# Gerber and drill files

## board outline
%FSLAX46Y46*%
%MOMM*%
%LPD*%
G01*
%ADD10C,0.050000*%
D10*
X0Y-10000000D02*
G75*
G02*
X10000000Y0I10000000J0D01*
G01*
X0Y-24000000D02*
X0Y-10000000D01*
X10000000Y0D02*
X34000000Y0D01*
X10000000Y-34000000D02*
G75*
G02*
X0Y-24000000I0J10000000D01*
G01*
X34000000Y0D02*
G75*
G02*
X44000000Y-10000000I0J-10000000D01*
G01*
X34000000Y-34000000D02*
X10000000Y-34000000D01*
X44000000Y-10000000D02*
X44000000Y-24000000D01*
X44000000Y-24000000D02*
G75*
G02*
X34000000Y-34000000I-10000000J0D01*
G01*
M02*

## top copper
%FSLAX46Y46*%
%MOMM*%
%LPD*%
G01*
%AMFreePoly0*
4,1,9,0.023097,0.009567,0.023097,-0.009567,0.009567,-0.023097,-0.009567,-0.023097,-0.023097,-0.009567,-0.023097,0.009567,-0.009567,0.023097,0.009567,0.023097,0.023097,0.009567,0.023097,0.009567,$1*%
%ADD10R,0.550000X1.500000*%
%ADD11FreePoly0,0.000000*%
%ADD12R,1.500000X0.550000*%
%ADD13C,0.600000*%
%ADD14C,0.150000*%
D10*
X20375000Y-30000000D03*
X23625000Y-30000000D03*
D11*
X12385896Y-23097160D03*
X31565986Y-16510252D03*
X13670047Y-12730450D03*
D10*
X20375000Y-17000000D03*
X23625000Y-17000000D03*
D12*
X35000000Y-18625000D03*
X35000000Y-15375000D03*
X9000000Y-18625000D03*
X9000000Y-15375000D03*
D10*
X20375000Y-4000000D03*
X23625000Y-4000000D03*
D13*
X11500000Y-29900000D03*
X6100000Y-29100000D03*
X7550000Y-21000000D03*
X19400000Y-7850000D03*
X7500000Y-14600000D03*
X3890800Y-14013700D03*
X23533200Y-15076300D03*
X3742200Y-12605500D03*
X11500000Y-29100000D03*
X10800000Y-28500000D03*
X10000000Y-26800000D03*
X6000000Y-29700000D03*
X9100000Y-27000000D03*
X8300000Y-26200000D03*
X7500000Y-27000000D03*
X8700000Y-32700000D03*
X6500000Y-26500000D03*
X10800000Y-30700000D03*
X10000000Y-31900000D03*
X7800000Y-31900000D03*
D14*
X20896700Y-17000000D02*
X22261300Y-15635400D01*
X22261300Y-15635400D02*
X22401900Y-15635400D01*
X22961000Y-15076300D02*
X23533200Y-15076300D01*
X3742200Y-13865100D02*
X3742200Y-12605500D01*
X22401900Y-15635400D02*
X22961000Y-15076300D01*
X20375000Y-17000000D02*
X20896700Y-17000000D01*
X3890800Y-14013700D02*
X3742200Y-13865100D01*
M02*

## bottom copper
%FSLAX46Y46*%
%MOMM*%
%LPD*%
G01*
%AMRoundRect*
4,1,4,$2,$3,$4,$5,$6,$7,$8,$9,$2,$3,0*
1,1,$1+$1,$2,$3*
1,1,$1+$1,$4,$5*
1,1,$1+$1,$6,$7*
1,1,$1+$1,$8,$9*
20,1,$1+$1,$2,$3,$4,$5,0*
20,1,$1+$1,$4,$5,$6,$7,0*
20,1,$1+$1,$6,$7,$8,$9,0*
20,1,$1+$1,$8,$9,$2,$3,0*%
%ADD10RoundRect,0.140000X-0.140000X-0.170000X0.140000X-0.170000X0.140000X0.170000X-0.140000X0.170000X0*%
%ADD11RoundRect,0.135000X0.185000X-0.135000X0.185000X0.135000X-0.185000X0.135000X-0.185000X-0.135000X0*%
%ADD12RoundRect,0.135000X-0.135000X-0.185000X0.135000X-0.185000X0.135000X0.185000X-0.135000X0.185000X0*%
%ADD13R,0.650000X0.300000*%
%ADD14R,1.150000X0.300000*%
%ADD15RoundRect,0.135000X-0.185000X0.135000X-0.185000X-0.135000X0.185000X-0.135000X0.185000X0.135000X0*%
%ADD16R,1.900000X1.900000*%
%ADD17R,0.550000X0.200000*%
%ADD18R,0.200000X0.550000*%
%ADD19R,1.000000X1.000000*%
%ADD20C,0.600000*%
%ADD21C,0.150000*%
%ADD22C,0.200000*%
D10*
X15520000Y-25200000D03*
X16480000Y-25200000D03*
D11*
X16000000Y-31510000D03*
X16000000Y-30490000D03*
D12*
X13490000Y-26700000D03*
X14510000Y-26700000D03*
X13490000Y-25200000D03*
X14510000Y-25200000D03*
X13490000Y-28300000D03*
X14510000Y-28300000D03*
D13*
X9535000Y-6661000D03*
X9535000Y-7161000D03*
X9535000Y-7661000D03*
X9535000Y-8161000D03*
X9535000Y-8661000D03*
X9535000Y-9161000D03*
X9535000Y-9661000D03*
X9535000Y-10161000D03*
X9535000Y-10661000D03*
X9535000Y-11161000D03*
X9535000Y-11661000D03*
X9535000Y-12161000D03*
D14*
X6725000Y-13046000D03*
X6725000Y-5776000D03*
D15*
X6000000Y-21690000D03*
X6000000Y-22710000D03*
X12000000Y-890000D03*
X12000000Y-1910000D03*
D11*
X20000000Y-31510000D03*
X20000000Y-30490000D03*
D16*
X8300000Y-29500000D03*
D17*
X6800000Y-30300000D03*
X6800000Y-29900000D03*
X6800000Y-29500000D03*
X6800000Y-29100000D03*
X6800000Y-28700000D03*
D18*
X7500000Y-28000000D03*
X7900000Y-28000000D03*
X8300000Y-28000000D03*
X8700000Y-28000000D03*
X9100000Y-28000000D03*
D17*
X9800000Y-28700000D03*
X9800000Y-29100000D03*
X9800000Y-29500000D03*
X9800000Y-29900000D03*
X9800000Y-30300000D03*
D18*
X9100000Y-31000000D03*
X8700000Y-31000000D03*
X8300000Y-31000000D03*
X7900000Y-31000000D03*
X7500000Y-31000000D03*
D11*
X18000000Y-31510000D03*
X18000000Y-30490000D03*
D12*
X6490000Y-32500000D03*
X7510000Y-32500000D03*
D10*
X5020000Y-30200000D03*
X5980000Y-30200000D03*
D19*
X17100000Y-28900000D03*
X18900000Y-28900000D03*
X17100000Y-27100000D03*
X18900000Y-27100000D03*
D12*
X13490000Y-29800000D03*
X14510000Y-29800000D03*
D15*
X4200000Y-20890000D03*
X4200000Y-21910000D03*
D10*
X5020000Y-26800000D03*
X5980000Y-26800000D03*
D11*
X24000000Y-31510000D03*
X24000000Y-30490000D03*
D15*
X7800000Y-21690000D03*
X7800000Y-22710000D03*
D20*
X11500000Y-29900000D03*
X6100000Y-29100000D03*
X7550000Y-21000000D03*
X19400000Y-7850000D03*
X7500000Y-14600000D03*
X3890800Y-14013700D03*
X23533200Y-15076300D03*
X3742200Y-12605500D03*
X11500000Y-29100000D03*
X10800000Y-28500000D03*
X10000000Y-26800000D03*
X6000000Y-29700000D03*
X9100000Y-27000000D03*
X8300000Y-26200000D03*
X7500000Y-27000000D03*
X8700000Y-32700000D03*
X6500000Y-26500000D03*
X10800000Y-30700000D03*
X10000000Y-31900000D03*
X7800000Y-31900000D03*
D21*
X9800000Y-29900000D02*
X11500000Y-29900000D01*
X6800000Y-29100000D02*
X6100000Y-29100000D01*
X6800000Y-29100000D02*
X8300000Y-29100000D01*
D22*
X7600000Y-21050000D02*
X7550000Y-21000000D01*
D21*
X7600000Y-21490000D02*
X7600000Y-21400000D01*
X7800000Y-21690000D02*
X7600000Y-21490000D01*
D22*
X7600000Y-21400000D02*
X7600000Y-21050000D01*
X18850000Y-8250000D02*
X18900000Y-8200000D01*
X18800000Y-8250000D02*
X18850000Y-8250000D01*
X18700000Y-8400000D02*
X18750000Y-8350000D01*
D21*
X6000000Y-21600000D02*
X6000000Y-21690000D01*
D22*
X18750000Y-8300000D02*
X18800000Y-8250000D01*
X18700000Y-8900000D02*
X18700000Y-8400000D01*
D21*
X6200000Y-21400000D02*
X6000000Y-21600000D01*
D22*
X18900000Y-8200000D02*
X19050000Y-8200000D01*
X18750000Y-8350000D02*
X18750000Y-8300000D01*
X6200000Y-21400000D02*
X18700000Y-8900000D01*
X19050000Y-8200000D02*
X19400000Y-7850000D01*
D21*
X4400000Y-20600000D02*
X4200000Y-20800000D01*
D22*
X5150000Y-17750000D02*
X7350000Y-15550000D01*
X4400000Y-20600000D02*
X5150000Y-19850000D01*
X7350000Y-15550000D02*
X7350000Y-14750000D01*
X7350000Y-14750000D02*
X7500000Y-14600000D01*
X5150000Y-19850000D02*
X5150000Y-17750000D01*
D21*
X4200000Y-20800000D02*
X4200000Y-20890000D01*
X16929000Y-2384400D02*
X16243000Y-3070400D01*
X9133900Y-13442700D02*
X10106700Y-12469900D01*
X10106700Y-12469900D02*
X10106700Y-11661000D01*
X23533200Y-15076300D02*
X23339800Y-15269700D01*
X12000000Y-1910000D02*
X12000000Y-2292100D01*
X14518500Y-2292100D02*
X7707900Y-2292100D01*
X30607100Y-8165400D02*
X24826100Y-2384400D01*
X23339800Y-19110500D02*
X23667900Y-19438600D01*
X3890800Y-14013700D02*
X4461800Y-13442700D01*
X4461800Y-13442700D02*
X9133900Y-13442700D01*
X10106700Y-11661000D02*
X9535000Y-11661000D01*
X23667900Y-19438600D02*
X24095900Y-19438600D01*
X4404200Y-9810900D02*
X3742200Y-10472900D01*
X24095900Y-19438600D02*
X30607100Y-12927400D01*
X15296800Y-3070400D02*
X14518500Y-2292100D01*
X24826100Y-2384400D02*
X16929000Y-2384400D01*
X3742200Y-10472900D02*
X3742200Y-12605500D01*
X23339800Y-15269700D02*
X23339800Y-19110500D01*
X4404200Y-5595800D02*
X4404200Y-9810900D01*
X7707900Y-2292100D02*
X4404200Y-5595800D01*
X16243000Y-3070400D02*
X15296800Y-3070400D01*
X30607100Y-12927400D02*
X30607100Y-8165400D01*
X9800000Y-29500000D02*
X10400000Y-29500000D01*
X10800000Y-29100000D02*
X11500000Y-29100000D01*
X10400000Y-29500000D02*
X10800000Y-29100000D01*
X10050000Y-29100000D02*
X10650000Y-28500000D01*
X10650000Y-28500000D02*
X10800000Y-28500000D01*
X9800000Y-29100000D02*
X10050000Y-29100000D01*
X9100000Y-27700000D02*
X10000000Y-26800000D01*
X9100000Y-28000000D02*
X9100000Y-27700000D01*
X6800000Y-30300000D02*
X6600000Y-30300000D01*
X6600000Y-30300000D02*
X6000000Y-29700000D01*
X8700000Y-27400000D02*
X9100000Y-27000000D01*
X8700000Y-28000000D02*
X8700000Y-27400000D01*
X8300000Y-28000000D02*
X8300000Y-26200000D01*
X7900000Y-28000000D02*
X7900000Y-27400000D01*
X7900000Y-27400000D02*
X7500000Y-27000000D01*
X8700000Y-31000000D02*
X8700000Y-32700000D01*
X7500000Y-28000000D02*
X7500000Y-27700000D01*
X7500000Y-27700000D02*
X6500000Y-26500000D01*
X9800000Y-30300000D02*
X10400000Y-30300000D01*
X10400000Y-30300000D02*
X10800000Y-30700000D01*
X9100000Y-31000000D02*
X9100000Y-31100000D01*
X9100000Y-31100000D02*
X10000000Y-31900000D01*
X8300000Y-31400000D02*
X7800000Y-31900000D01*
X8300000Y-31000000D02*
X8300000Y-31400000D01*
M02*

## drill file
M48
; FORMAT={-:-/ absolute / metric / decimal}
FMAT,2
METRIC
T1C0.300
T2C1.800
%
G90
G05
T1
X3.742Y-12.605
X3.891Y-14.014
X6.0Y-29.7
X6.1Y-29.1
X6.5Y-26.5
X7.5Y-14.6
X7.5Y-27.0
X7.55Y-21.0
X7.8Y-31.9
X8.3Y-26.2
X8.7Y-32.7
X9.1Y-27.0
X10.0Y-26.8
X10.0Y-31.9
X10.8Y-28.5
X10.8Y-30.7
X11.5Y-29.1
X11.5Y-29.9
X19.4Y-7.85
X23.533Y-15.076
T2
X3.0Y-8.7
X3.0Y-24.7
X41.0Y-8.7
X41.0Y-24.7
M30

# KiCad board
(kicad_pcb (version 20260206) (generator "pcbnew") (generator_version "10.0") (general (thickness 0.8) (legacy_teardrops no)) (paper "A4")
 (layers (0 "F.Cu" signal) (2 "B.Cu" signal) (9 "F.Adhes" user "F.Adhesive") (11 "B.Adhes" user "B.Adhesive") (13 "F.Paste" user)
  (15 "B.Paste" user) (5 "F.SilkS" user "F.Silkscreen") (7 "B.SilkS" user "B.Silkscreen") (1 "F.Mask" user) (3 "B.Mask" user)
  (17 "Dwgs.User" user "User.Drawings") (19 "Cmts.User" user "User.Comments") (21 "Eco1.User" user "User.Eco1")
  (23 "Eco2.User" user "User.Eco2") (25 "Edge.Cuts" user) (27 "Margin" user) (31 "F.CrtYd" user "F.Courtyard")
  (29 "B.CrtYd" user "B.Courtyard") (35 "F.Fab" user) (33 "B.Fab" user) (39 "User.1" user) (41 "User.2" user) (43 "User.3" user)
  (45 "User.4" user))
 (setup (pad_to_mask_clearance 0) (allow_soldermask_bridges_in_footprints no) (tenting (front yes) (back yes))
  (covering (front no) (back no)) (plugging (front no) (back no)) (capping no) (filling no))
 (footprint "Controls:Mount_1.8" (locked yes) (layer "F.Cu") (at 41 24.7)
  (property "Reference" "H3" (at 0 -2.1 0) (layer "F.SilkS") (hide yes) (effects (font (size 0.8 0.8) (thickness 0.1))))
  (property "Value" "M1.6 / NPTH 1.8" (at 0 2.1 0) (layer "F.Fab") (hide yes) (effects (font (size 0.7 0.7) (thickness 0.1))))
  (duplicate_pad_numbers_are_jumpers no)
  (pad "" np_thru_hole circle (at 0 0) (size 1.8 1.8) (drill 1.8) (layers "*.Cu" "*.Mask")))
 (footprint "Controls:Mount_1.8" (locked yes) (layer "F.Cu") (at 3 8.7)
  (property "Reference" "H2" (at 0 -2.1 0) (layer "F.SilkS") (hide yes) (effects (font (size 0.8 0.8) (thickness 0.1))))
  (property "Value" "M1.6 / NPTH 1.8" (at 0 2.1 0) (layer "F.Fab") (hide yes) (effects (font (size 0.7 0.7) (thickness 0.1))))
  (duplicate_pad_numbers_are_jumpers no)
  (pad "" np_thru_hole circle (at 0 0) (size 1.8 1.8) (drill 1.8) (layers "*.Cu" "*.Mask")))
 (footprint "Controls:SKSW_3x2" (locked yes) (layer "F.Cu") (at 22 30)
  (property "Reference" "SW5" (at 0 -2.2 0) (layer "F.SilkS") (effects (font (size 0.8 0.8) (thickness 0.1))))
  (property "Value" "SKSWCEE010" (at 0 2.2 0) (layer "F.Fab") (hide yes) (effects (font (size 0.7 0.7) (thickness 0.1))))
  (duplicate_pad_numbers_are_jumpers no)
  (pad "1" smd rect (at -1.625 0) (size 0.55 1.5) (layers "F.Cu" "F.Mask" "F.Paste") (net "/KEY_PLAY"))
  (pad "2" smd rect (at 1.625 0) (size 0.55 1.5) (layers "F.Cu" "F.Mask" "F.Paste") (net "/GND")))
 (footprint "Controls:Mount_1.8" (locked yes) (layer "F.Cu") (at 41 8.7)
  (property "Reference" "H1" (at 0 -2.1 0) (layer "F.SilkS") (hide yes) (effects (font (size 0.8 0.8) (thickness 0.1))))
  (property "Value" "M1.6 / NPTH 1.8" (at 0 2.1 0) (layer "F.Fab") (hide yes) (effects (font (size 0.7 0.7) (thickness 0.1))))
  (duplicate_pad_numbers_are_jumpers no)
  (pad "" np_thru_hole circle (at 0 0) (size 1.8 1.8) (drill 1.8) (layers "*.Cu" "*.Mask")))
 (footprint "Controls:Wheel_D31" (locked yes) (layer "F.Cu") (at 22 17)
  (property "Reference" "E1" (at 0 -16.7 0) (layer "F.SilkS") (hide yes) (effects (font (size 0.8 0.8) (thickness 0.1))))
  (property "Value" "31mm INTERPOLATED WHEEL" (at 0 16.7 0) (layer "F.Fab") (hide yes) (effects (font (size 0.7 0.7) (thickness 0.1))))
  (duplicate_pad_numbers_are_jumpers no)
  (pad "1" smd custom (at -9.614104 6.09716) (size 0.05 0.05) (layers "F.Cu") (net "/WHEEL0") (options (clearance outline) (anchor circle))
   (primitives))
  (pad "2" smd custom (at 9.565986 -0.489748) (size 0.05 0.05) (layers "F.Cu") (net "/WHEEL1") (options (clearance outline) (anchor circle))
   (primitives))
  (pad "3" smd custom (at -8.329953 -4.26955) (size 0.05 0.05) (layers "F.Cu") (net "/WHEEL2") (options (clearance outline) (anchor circle))
   (primitives)))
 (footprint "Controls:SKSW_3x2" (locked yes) (layer "F.Cu") (at 22 17)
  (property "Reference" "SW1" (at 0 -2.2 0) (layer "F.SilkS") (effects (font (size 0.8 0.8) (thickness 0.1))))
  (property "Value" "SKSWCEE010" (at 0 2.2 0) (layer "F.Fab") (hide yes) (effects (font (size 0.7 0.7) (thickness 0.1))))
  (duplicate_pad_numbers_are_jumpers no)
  (pad "1" smd rect (at -1.625 0) (size 0.55 1.5) (layers "F.Cu" "F.Mask" "F.Paste") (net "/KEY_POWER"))
  (pad "2" smd rect (at 1.625 0) (size 0.55 1.5) (layers "F.Cu" "F.Mask" "F.Paste") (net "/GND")))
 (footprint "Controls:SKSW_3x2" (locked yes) (layer "F.Cu") (at 35 17 90)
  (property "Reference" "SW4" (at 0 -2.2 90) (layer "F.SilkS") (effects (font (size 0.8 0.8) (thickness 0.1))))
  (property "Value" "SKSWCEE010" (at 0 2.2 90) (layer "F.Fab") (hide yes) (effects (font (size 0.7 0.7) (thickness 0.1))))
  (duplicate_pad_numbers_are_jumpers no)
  (pad "1" smd rect (at -1.625 0 90) (size 0.55 1.5) (layers "F.Cu" "F.Mask" "F.Paste") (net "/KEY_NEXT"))
  (pad "2" smd rect (at 1.625 0 90) (size 0.55 1.5) (layers "F.Cu" "F.Mask" "F.Paste") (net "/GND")))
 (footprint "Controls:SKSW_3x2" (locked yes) (layer "F.Cu") (at 9 17 90)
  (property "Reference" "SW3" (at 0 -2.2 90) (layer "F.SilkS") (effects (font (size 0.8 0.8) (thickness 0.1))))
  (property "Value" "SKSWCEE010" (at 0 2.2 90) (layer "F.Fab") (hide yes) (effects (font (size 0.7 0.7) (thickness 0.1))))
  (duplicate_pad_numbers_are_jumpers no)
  (pad "1" smd rect (at -1.625 0 90) (size 0.55 1.5) (layers "F.Cu" "F.Mask" "F.Paste") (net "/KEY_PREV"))
  (pad "2" smd rect (at 1.625 0 90) (size 0.55 1.5) (layers "F.Cu" "F.Mask" "F.Paste") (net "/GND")))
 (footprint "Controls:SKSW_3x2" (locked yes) (layer "F.Cu") (at 22 4)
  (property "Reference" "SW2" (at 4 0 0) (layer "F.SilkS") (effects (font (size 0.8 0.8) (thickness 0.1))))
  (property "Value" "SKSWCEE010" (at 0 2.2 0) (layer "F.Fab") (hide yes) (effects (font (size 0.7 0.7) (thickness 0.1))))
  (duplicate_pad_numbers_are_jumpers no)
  (pad "1" smd rect (at -1.625 0) (size 0.55 1.5) (layers "F.Cu" "F.Mask" "F.Paste") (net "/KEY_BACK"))
  (pad "2" smd rect (at 1.625 0) (size 0.55 1.5) (layers "F.Cu" "F.Mask" "F.Paste") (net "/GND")))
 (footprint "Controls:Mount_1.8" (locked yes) (layer "F.Cu") (at 3 24.7)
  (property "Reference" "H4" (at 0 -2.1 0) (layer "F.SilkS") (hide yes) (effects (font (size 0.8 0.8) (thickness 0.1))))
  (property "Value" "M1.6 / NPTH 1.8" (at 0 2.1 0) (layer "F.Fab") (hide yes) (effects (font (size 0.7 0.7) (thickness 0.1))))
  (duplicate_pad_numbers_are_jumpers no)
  (pad "" np_thru_hole circle (at 0 0) (size 1.8 1.8) (drill 1.8) (layers "*.Cu" "*.Mask")))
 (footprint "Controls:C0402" (layer "B.Cu") (at 16 25.2)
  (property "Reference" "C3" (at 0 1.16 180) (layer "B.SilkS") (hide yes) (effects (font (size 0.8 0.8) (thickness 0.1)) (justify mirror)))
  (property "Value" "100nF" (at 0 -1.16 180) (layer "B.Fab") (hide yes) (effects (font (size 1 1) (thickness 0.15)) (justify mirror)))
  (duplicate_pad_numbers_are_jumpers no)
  (pad "1" smd roundrect (at -0.48 0) (size 0.56 0.62) (layers "B.Cu" "B.Mask" "B.Paste") (roundrect_rratio 0.25) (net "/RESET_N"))
  (pad "2" smd roundrect (at 0.48 0) (size 0.56 0.62) (layers "B.Cu" "B.Mask" "B.Paste") (roundrect_rratio 0.25) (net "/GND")))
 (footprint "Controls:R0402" (layer "B.Cu") (at 16 31 90)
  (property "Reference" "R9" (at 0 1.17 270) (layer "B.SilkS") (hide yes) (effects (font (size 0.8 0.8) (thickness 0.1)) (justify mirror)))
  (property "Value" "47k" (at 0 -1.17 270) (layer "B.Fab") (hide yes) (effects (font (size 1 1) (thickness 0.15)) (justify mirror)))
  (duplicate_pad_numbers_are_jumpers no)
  (pad "1" smd roundrect (at -0.51 0 90) (size 0.54 0.64) (layers "B.Cu" "B.Mask" "B.Paste") (roundrect_rratio 0.25) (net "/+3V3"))
  (pad "2" smd roundrect (at 0.51 0 90) (size 0.54 0.64) (layers "B.Cu" "B.Mask" "B.Paste") (roundrect_rratio 0.25) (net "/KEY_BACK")))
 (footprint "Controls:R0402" (layer "B.Cu") (at 14 26.7)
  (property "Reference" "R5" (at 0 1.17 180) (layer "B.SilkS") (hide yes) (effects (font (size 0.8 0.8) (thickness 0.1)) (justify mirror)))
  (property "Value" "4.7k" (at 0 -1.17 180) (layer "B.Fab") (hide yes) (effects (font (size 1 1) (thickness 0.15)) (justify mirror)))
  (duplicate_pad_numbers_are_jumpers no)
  (pad "1" smd roundrect (at -0.51 0) (size 0.54 0.64) (layers "B.Cu" "B.Mask" "B.Paste") (roundrect_rratio 0.25) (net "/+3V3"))
  (pad "2" smd roundrect (at 0.51 0) (size 0.54 0.64) (layers "B.Cu" "B.Mask" "B.Paste") (roundrect_rratio 0.25) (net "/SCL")))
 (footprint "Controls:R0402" (layer "B.Cu") (at 14 25.2)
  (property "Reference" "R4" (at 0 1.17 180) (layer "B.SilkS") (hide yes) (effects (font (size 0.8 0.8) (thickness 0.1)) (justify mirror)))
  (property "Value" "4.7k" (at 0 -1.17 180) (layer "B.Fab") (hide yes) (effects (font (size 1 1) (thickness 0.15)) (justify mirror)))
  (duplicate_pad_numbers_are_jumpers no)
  (pad "1" smd roundrect (at -0.51 0) (size 0.54 0.64) (layers "B.Cu" "B.Mask" "B.Paste") (roundrect_rratio 0.25) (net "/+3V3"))
  (pad "2" smd roundrect (at 0.51 0) (size 0.54 0.64) (layers "B.Cu" "B.Mask" "B.Paste") (roundrect_rratio 0.25) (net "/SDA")))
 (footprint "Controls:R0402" (layer "B.Cu") (at 14 28.3)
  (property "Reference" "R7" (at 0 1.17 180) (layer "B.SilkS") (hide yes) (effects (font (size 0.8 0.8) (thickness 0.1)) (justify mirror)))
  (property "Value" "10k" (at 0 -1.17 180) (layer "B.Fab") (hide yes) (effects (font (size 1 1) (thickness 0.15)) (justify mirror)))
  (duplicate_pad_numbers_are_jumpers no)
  (pad "1" smd roundrect (at -0.51 0) (size 0.54 0.64) (layers "B.Cu" "B.Mask" "B.Paste") (roundrect_rratio 0.25) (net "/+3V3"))
  (pad "2" smd roundrect (at 0.51 0) (size 0.54 0.64) (layers "B.Cu" "B.Mask" "B.Paste") (roundrect_rratio 0.25) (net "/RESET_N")))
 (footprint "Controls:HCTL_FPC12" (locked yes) (layer "B.Cu") (at 8.13 9.411 -90)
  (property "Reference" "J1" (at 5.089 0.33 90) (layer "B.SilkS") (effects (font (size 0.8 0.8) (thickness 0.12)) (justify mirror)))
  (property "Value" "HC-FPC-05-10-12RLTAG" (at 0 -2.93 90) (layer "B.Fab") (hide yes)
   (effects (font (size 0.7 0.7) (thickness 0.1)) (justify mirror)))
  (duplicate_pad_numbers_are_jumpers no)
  (pad "1" smd rect (at -2.75 -1.405 270) (size 0.3 0.65) (layers "B.Cu" "B.Mask" "B.Paste") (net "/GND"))
  (pad "2" smd rect (at -2.25 -1.405 270) (size 0.3 0.65) (layers "B.Cu" "B.Mask" "B.Paste") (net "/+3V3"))
  (pad "3" smd rect (at -1.75 -1.405 270) (size 0.3 0.65) (layers "B.Cu" "B.Mask" "B.Paste") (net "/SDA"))
  (pad "4" smd rect (at -1.25 -1.405 270) (size 0.3 0.65) (layers "B.Cu" "B.Mask" "B.Paste") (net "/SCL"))
  (pad "5" smd rect (at -0.75 -1.405 270) (size 0.3 0.65) (layers "B.Cu" "B.Mask" "B.Paste") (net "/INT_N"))
  (pad "6" smd rect (at -0.25 -1.405 270) (size 0.3 0.65) (layers "B.Cu" "B.Mask" "B.Paste") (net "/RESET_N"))
  (pad "7" smd rect (at 0.25 -1.405 270) (size 0.3 0.65) (layers "B.Cu" "B.Mask" "B.Paste") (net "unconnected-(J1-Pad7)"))
  (pad "8" smd rect (at 0.75 -1.405 270) (size 0.3 0.65) (layers "B.Cu" "B.Mask" "B.Paste") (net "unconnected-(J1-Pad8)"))
  (pad "9" smd rect (at 1.25 -1.405 270) (size 0.3 0.65) (layers "B.Cu" "B.Mask" "B.Paste") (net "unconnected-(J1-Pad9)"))
  (pad "10" smd rect (at 1.75 -1.405 270) (size 0.3 0.65) (layers "B.Cu" "B.Mask" "B.Paste") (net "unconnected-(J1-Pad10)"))
  (pad "11" smd rect (at 2.25 -1.405 270) (size 0.3 0.65) (layers "B.Cu" "B.Mask" "B.Paste") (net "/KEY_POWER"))
  (pad "12" smd rect (at 2.75 -1.405 270) (size 0.3 0.65) (layers "B.Cu" "B.Mask" "B.Paste") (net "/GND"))
  (pad "13" smd rect (at 3.635 1.405 270) (size 0.3 1.15) (layers "B.Cu" "B.Mask" "B.Paste") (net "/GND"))
  (pad "14" smd rect (at -3.635 1.405 270) (size 0.3 1.15) (layers "B.Cu" "B.Mask" "B.Paste") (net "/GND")))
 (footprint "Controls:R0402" (layer "B.Cu") (at 6 22.2 -90)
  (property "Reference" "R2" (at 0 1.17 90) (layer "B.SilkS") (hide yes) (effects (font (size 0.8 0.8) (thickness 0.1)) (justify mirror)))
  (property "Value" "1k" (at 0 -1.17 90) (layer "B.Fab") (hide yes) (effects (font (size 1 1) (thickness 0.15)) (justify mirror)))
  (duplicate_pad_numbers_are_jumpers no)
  (pad "1" smd roundrect (at -0.51 0 270) (size 0.54 0.64) (layers "B.Cu" "B.Mask" "B.Paste") (roundrect_rratio 0.25) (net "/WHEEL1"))
  (pad "2" smd roundrect (at 0.51 0 270) (size 0.54 0.64) (layers "B.Cu" "B.Mask" "B.Paste") (roundrect_rratio 0.25) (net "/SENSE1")))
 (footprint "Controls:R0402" (layer "B.Cu") (at 12 1.4 -90)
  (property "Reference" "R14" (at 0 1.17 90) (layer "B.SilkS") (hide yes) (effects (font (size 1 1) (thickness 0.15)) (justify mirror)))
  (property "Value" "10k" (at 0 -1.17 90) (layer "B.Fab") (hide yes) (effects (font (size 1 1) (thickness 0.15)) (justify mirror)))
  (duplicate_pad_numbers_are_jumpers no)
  (pad "1" smd roundrect (at -0.51 0 270) (size 0.54 0.64) (layers "B.Cu" "B.Mask" "B.Paste") (roundrect_rratio 0.25) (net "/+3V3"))
  (pad "2" smd roundrect (at 0.51 0 270) (size 0.54 0.64) (layers "B.Cu" "B.Mask" "B.Paste") (roundrect_rratio 0.25) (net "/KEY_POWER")))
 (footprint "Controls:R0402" (layer "B.Cu") (at 20 31 90)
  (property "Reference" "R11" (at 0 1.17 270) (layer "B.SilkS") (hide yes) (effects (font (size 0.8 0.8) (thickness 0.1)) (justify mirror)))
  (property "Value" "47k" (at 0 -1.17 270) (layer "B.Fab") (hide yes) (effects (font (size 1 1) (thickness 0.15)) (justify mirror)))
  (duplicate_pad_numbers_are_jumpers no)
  (pad "1" smd roundrect (at -0.51 0 90) (size 0.54 0.64) (layers "B.Cu" "B.Mask" "B.Paste") (roundrect_rratio 0.25) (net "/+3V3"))
  (pad "2" smd roundrect (at 0.51 0 90) (size 0.54 0.64) (layers "B.Cu" "B.Mask" "B.Paste") (roundrect_rratio 0.25) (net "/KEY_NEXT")))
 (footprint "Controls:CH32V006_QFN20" (layer "B.Cu") (at 8.3 29.5)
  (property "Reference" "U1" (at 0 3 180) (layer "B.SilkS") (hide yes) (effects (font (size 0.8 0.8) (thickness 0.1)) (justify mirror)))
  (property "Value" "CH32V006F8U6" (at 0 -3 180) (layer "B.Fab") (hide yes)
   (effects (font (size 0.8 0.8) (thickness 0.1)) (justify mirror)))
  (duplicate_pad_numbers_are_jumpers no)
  (pad "" smd rect (at -0.45 -0.45) (size 0.7 0.7) (layers "B.Paste"))
  (pad "" smd rect (at -0.45 0.45) (size 0.7 0.7) (layers "B.Paste"))
  (pad "" smd rect (at 0.45 -0.45) (size 0.7 0.7) (layers "B.Paste"))
  (pad "" smd rect (at 0.45 0.45) (size 0.7 0.7) (layers "B.Paste"))
  (pad "0" smd rect (at 0 0) (size 1.9 1.9) (layers "B.Cu" "B.Mask") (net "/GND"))
  (pad "1" smd rect (at -1.5 0.8) (size 0.55 0.2) (layers "B.Cu" "B.Mask" "B.Paste") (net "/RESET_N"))
  (pad "2" smd rect (at -1.5 0.4) (size 0.55 0.2) (layers "B.Cu" "B.Mask" "B.Paste") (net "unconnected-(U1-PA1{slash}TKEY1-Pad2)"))
  (pad "3" smd rect (at -1.5 0) (size 0.55 0.2) (layers "B.Cu" "B.Mask" "B.Paste") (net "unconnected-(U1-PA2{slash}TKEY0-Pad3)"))
  (pad "4" smd rect (at -1.5 -0.4) (size 0.55 0.2) (layers "B.Cu" "B.Mask" "B.Paste") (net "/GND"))
  (pad "5" smd rect (at -1.5 -0.8) (size 0.55 0.2) (layers "B.Cu" "B.Mask" "B.Paste") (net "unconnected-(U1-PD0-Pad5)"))
  (pad "6" smd rect (at -0.8 -1.5) (size 0.2 0.55) (layers "B.Cu" "B.Mask" "B.Paste") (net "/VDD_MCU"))
  (pad "7" smd rect (at -0.4 -1.5) (size 0.2 0.55) (layers "B.Cu" "B.Mask" "B.Paste") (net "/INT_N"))
  (pad "8" smd rect (at 0 -1.5) (size 0.2 0.55) (layers "B.Cu" "B.Mask" "B.Paste") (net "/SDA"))
  (pad "9" smd rect (at 0.4 -1.5) (size 0.2 0.55) (layers "B.Cu" "B.Mask" "B.Paste") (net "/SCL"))
  (pad "10" smd rect (at 0.8 -1.5) (size 0.2 0.55) (layers "B.Cu" "B.Mask" "B.Paste") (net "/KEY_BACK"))
  (pad "11" smd rect (at 1.5 -0.8) (size 0.55 0.2) (layers "B.Cu" "B.Mask" "B.Paste") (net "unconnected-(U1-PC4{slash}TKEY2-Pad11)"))
  (pad "12" smd rect (at 1.5 -0.4) (size 0.55 0.2) (layers "B.Cu" "B.Mask" "B.Paste") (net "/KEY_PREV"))
  (pad "13" smd rect (at 1.5 0) (size 0.55 0.2) (layers "B.Cu" "B.Mask" "B.Paste") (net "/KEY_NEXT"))
  (pad "14" smd rect (at 1.5 0.4) (size 0.55 0.2) (layers "B.Cu" "B.Mask" "B.Paste") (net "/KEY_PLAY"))
  (pad "15" smd rect (at 1.5 0.8) (size 0.55 0.2) (layers "B.Cu" "B.Mask" "B.Paste") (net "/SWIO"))
  (pad "16" smd rect (at 0.8 1.5) (size 0.2 0.55) (layers "B.Cu" "B.Mask" "B.Paste") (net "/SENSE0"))
  (pad "17" smd rect (at 0.4 1.5) (size 0.2 0.55) (layers "B.Cu" "B.Mask" "B.Paste") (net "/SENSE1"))
  (pad "18" smd rect (at 0 1.5) (size 0.2 0.55) (layers "B.Cu" "B.Mask" "B.Paste") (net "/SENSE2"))
  (pad "19" smd rect (at -0.4 1.5) (size 0.2 0.55) (layers "B.Cu" "B.Mask" "B.Paste") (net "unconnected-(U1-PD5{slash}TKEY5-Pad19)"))
  (pad "20" smd rect (at -0.8 1.5) (size 0.2 0.55) (layers "B.Cu" "B.Mask" "B.Paste") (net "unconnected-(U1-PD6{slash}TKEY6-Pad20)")))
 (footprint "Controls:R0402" (layer "B.Cu") (at 18 31 90)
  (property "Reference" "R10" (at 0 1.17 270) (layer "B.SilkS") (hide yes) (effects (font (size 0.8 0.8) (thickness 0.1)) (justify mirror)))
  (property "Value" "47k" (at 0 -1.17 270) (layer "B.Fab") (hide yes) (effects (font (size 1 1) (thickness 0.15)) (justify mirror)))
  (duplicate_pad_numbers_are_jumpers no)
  (pad "1" smd roundrect (at -0.51 0 90) (size 0.54 0.64) (layers "B.Cu" "B.Mask" "B.Paste") (roundrect_rratio 0.25) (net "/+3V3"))
  (pad "2" smd roundrect (at 0.51 0 90) (size 0.54 0.64) (layers "B.Cu" "B.Mask" "B.Paste") (roundrect_rratio 0.25) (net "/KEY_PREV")))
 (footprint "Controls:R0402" (layer "B.Cu") (at 7 32.5)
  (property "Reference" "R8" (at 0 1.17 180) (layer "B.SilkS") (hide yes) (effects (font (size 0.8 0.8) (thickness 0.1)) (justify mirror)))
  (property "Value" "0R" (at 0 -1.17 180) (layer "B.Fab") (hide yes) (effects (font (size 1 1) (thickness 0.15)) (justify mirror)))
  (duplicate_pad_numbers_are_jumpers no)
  (pad "1" smd roundrect (at -0.51 0) (size 0.54 0.64) (layers "B.Cu" "B.Mask" "B.Paste") (roundrect_rratio 0.25) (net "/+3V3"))
  (pad "2" smd roundrect (at 0.51 0) (size 0.54 0.64) (layers "B.Cu" "B.Mask" "B.Paste") (roundrect_rratio 0.25) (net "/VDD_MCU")))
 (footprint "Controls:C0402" (layer "B.Cu") (at 5.5 30.2)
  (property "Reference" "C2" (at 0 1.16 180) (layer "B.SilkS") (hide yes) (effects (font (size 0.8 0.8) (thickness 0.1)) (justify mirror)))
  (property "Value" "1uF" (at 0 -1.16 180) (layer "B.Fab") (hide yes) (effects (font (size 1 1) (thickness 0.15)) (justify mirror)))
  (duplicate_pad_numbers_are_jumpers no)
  (pad "1" smd roundrect (at -0.48 0) (size 0.56 0.62) (layers "B.Cu" "B.Mask" "B.Paste") (roundrect_rratio 0.25) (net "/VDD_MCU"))
  (pad "2" smd roundrect (at 0.48 0) (size 0.56 0.62) (layers "B.Cu" "B.Mask" "B.Paste") (roundrect_rratio 0.25) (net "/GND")))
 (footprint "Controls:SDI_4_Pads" (layer "B.Cu") (at 18 28)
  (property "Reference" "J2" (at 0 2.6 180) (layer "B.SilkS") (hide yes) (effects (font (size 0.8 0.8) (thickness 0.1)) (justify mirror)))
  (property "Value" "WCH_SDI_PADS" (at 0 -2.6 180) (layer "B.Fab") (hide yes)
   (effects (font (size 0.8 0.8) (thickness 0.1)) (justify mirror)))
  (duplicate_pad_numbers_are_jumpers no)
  (pad "1" smd rect (at -0.9 0.9) (size 1 1) (layers "B.Cu" "B.Mask") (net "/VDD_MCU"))
  (pad "2" smd rect (at 0.9 0.9) (size 1 1) (layers "B.Cu" "B.Mask") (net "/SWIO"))
  (pad "3" smd rect (at -0.9 -0.9) (size 1 1) (layers "B.Cu" "B.Mask") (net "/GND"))
  (pad "4" smd rect (at 0.9 -0.9) (size 1 1) (layers "B.Cu" "B.Mask") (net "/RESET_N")))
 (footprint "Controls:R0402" (layer "B.Cu") (at 14 29.8)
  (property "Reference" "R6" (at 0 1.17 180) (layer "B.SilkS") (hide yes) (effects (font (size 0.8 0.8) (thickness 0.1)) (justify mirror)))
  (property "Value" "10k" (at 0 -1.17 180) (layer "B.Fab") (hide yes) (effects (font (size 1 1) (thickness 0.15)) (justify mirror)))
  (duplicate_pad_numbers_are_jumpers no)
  (pad "1" smd roundrect (at -0.51 0) (size 0.54 0.64) (layers "B.Cu" "B.Mask" "B.Paste") (roundrect_rratio 0.25) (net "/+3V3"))
  (pad "2" smd roundrect (at 0.51 0) (size 0.54 0.64) (layers "B.Cu" "B.Mask" "B.Paste") (roundrect_rratio 0.25) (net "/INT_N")))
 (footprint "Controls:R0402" (layer "B.Cu") (at 4.2 21.4 -90)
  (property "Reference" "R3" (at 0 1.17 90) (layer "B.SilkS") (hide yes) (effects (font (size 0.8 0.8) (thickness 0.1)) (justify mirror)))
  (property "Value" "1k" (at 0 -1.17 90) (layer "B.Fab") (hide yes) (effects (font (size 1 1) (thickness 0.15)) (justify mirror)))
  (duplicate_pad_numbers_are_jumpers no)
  (pad "1" smd roundrect (at -0.51 0 270) (size 0.54 0.64) (layers "B.Cu" "B.Mask" "B.Paste") (roundrect_rratio 0.25) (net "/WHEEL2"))
  (pad "2" smd roundrect (at 0.51 0 270) (size 0.54 0.64) (layers "B.Cu" "B.Mask" "B.Paste") (roundrect_rratio 0.25) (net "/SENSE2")))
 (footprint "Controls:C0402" (layer "B.Cu") (at 5.5 26.8)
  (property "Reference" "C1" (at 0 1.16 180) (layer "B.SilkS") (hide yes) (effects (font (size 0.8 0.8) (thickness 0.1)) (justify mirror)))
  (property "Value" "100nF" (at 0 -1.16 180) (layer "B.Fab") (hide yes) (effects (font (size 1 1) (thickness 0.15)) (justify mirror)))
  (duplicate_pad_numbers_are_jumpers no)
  (pad "1" smd roundrect (at -0.48 0) (size 0.56 0.62) (layers "B.Cu" "B.Mask" "B.Paste") (roundrect_rratio 0.25) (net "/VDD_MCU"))
  (pad "2" smd roundrect (at 0.48 0) (size 0.56 0.62) (layers "B.Cu" "B.Mask" "B.Paste") (roundrect_rratio 0.25) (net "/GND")))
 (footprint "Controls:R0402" (layer "B.Cu") (at 24 31 90)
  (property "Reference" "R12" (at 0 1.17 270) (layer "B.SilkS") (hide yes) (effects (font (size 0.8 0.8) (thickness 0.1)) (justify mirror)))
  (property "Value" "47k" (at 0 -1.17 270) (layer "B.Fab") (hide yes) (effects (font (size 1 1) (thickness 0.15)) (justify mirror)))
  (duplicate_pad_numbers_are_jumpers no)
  (pad "1" smd roundrect (at -0.51 0 90) (size 0.54 0.64) (layers "B.Cu" "B.Mask" "B.Paste") (roundrect_rratio 0.25) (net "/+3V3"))
  (pad "2" smd roundrect (at 0.51 0 90) (size 0.54 0.64) (layers "B.Cu" "B.Mask" "B.Paste") (roundrect_rratio 0.25) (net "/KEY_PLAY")))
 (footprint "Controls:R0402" (layer "B.Cu") (at 7.8 22.2 -90)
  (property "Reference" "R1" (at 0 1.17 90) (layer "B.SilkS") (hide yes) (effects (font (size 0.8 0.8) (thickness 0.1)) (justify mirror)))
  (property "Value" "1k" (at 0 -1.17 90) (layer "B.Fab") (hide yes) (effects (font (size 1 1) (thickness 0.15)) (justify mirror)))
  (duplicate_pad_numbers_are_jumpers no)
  (pad "1" smd roundrect (at -0.51 0 270) (size 0.54 0.64) (layers "B.Cu" "B.Mask" "B.Paste") (roundrect_rratio 0.25) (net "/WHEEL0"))
  (pad "2" smd roundrect (at 0.51 0 270) (size 0.54 0.64) (layers "B.Cu" "B.Mask" "B.Paste") (roundrect_rratio 0.25) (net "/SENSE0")))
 (gr_arc (start 0 10) (mid 2.928932 2.928932) (end 10 0) (stroke (width 0.05) (type default)) (layer "Edge.Cuts"))
 (gr_line (start 0 24) (end 0 10) (stroke (width 0.05) (type default)) (layer "Edge.Cuts"))
 (gr_line (start 10 0) (end 34 0) (stroke (width 0.05) (type default)) (layer "Edge.Cuts"))
 (gr_arc (start 10 34) (mid 2.928932 31.071068) (end 0 24) (stroke (width 0.05) (type default)) (layer "Edge.Cuts"))
 (gr_arc (start 34 0) (mid 41.071068 2.928932) (end 44 10) (stroke (width 0.05) (type default)) (layer "Edge.Cuts"))
 (gr_line (start 34 34) (end 10 34) (stroke (width 0.05) (type default)) (layer "Edge.Cuts"))
 (gr_line (start 44 10) (end 44 24) (stroke (width 0.05) (type default)) (layer "Edge.Cuts"))
 (gr_arc (start 44 24) (mid 41.071068 31.071068) (end 34 34) (stroke (width 0.05) (type default)) (layer "Edge.Cuts"))
 (via (at 11.5 29.9) (size 0.6) (drill 0.3) (layers "F.Cu" "B.Cu") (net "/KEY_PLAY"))
 (segment (start 9.8 29.9) (end 11.5 29.9) (width 0.15) (layer "B.Cu") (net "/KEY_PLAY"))
 (via (at 6.1 29.1) (size 0.6) (drill 0.3) (layers "F.Cu" "B.Cu") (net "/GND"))
 (segment (start 6.8 29.1) (end 6.1 29.1) (width 0.15) (layer "B.Cu") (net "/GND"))
 (segment (start 6.8 29.1) (end 8.3 29.1) (width 0.15) (layer "B.Cu") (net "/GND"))
 (via (at 7.55 21) (size 0.6) (drill 0.3) (layers "F.Cu" "B.Cu") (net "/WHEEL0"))
 (segment (start 7.6 21.05) (end 7.55 21) (width 0.2) (layer "B.Cu") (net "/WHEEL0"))
 (segment (start 7.6 21.49) (end 7.6 21.4) (width 0.15) (layer "B.Cu") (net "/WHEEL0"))
 (segment (start 7.8 21.69) (end 7.6 21.49) (width 0.15) (layer "B.Cu") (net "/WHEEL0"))
 (segment (start 7.6 21.4) (end 7.6 21.05) (width 0.2) (layer "B.Cu") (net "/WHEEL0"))
 (via (at 19.4 7.85) (size 0.6) (drill 0.3) (layers "F.Cu" "B.Cu") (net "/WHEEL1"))
 (segment (start 18.85 8.25) (end 18.9 8.2) (width 0.2) (layer "B.Cu") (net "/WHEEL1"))
 (segment (start 18.8 8.25) (end 18.85 8.25) (width 0.2) (layer "B.Cu") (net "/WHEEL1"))
 (segment (start 18.7 8.4) (end 18.75 8.35) (width 0.2) (layer "B.Cu") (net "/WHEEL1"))
 (segment (start 6 21.6) (end 6 21.69) (width 0.15) (layer "B.Cu") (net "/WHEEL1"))
 (segment (start 18.75 8.3) (end 18.8 8.25) (width 0.2) (layer "B.Cu") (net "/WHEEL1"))
 (segment (start 18.7 8.9) (end 18.7 8.4) (width 0.2) (layer "B.Cu") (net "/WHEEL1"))
 (segment (start 6.2 21.4) (end 6 21.6) (width 0.15) (layer "B.Cu") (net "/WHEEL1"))
 (segment (start 18.9 8.2) (end 19.05 8.2) (width 0.2) (layer "B.Cu") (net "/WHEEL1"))
 (segment (start 18.75 8.35) (end 18.75 8.3) (width 0.2) (layer "B.Cu") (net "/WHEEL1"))
 (segment (start 6.2 21.4) (end 18.7 8.9) (width 0.2) (layer "B.Cu") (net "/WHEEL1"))
 (segment (start 19.05 8.2) (end 19.4 7.85) (width 0.2) (layer "B.Cu") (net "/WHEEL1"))
 (via (at 7.5 14.6) (size 0.6) (drill 0.3) (layers "F.Cu" "B.Cu") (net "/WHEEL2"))
 (segment (start 4.4 20.6) (end 4.2 20.8) (width 0.15) (layer "B.Cu") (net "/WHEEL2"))
 (segment (start 5.15 17.75) (end 7.35 15.55) (width 0.2) (layer "B.Cu") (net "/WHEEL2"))
 (segment (start 4.4 20.6) (end 5.15 19.85) (width 0.2) (layer "B.Cu") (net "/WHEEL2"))
 (segment (start 7.35 15.55) (end 7.35 14.75) (width 0.2) (layer "B.Cu") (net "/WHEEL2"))
 (segment (start 7.35 14.75) (end 7.5 14.6) (width 0.2) (layer "B.Cu") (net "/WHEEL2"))
 (segment (start 5.15 19.85) (end 5.15 17.75) (width 0.2) (layer "B.Cu") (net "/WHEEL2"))
 (segment (start 4.2 20.8) (end 4.2 20.89) (width 0.15) (layer "B.Cu") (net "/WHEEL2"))
 (segment (start 20.8967 17) (end 22.2613 15.6354) (width 0.15) (layer "F.Cu") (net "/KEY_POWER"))
 (segment (start 22.2613 15.6354) (end 22.4019 15.6354) (width 0.15) (layer "F.Cu") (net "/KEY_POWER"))
 (segment (start 22.961 15.0763) (end 23.5332 15.0763) (width 0.15) (layer "F.Cu") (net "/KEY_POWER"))
 (segment (start 3.7422 13.8651) (end 3.7422 12.6055) (width 0.15) (layer "F.Cu") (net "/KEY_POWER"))
 (segment (start 22.4019 15.6354) (end 22.961 15.0763) (width 0.15) (layer "F.Cu") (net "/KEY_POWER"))
 (segment (start 20.375 17) (end 20.8967 17) (width 0.15) (layer "F.Cu") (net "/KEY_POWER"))
 (segment (start 3.8908 14.0137) (end 3.7422 13.8651) (width 0.15) (layer "F.Cu") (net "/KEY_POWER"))
 (via (at 3.8908 14.0137) (size 0.6) (drill 0.3) (layers "F.Cu" "B.Cu") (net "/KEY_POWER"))
 (via (at 23.5332 15.0763) (size 0.6) (drill 0.3) (layers "F.Cu" "B.Cu") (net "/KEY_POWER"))
 (via (at 3.7422 12.6055) (size 0.6) (drill 0.3) (layers "F.Cu" "B.Cu") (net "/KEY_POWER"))
 (segment (start 16.929 2.3844) (end 16.243 3.0704) (width 0.15) (layer "B.Cu") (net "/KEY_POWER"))
 (segment (start 9.1339 13.4427) (end 10.1067 12.4699) (width 0.15) (layer "B.Cu") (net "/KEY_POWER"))
 (segment (start 10.1067 12.4699) (end 10.1067 11.661) (width 0.15) (layer "B.Cu") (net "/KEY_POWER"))
 (segment (start 23.5332 15.0763) (end 23.3398 15.2697) (width 0.15) (layer "B.Cu") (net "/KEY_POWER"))
 (segment (start 12 1.91) (end 12 2.2921) (width 0.15) (layer "B.Cu") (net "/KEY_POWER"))
 (segment (start 14.5185 2.2921) (end 7.7079 2.2921) (width 0.15) (layer "B.Cu") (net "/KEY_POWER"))
 (segment (start 30.6071 8.1654) (end 24.8261 2.3844) (width 0.15) (layer "B.Cu") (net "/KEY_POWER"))
 (segment (start 23.3398 19.1105) (end 23.6679 19.4386) (width 0.15) (layer "B.Cu") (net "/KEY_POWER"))
 (segment (start 3.8908 14.0137) (end 4.4618 13.4427) (width 0.15) (layer "B.Cu") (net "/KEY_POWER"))
 (segment (start 4.4618 13.4427) (end 9.1339 13.4427) (width 0.15) (layer "B.Cu") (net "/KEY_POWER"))
 (segment (start 10.1067 11.661) (end 9.535 11.661) (width 0.15) (layer "B.Cu") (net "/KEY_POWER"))
 (segment (start 23.6679 19.4386) (end 24.0959 19.4386) (width 0.15) (layer "B.Cu") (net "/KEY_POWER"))
 (segment (start 4.4042 9.8109) (end 3.7422 10.4729) (width 0.15) (layer "B.Cu") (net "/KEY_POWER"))
 (segment (start 24.0959 19.4386) (end 30.6071 12.9274) (width 0.15) (layer "B.Cu") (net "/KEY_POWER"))
 (segment (start 15.2968 3.0704) (end 14.5185 2.2921) (width 0.15) (layer "B.Cu") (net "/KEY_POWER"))
 (segment (start 24.8261 2.3844) (end 16.929 2.3844) (width 0.15) (layer "B.Cu") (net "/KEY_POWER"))
 (segment (start 3.7422 10.4729) (end 3.7422 12.6055) (width 0.15) (layer "B.Cu") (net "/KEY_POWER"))
 (segment (start 23.3398 15.2697) (end 23.3398 19.1105) (width 0.15) (layer "B.Cu") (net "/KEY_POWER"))
 (segment (start 4.4042 5.5958) (end 4.4042 9.8109) (width 0.15) (layer "B.Cu") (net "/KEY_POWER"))
 (segment (start 7.7079 2.2921) (end 4.4042 5.5958) (width 0.15) (layer "B.Cu") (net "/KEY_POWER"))
 (segment (start 16.243 3.0704) (end 15.2968 3.0704) (width 0.15) (layer "B.Cu") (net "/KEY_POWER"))
 (segment (start 30.6071 12.9274) (end 30.6071 8.1654) (width 0.15) (layer "B.Cu") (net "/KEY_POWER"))
 (via (at 11.5 29.1) (size 0.6) (drill 0.3) (layers "F.Cu" "B.Cu") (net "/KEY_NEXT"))
 (segment (start 9.8 29.5) (end 10.4 29.5) (width 0.15) (layer "B.Cu") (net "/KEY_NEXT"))
 (segment (start 10.8 29.1) (end 11.5 29.1) (width 0.15) (layer "B.Cu") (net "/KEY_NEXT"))
 (segment (start 10.4 29.5) (end 10.8 29.1) (width 0.15) (layer "B.Cu") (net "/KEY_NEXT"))
 (via (at 10.8 28.5) (size 0.6) (drill 0.3) (layers "F.Cu" "B.Cu") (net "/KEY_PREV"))
 (segment (start 10.05 29.1) (end 10.65 28.5) (width 0.15) (layer "B.Cu") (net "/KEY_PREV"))
 (segment (start 10.65 28.5) (end 10.8 28.5) (width 0.15) (layer "B.Cu") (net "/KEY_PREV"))
 (segment (start 9.8 29.1) (end 10.05 29.1) (width 0.15) (layer "B.Cu") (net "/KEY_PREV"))
 (via (at 10 26.8) (size 0.6) (drill 0.3) (layers "F.Cu" "B.Cu") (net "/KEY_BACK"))
 (segment (start 9.1 27.7) (end 10 26.8) (width 0.15) (layer "B.Cu") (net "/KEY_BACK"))
 (segment (start 9.1 28) (end 9.1 27.7) (width 0.15) (layer "B.Cu") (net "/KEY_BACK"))
 (via (at 6 29.7) (size 0.6) (drill 0.3) (layers "F.Cu" "B.Cu") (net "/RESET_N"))
 (segment (start 6.8 30.3) (end 6.6 30.3) (width 0.15) (layer "B.Cu") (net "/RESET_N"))
 (segment (start 6.6 30.3) (end 6 29.7) (width 0.15) (layer "B.Cu") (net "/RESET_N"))
 (via (at 9.1 27) (size 0.6) (drill 0.3) (layers "F.Cu" "B.Cu") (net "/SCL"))
 (segment (start 8.7 27.4) (end 9.1 27) (width 0.15) (layer "B.Cu") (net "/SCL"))
 (segment (start 8.7 28) (end 8.7 27.4) (width 0.15) (layer "B.Cu") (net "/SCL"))
 (via (at 8.3 26.2) (size 0.6) (drill 0.3) (layers "F.Cu" "B.Cu") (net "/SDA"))
 (segment (start 8.3 28) (end 8.3 26.2) (width 0.15) (layer "B.Cu") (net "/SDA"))
 (via (at 7.5 27) (size 0.6) (drill 0.3) (layers "F.Cu" "B.Cu") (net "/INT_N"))
 (segment (start 7.9 28) (end 7.9 27.4) (width 0.15) (layer "B.Cu") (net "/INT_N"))
 (segment (start 7.9 27.4) (end 7.5 27) (width 0.15) (layer "B.Cu") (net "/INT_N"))
 (via (at 8.7 32.7) (size 0.6) (drill 0.3) (layers "F.Cu" "B.Cu") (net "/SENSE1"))
 (segment (start 8.7 31) (end 8.7 32.7) (width 0.15) (layer "B.Cu") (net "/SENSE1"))
 (via (at 6.5 26.5) (size 0.6) (drill 0.3) (layers "F.Cu" "B.Cu") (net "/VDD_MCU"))
 (segment (start 7.5 28) (end 7.5 27.7) (width 0.15) (layer "B.Cu") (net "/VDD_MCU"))
 (segment (start 7.5 27.7) (end 6.5 26.5) (width 0.15) (layer "B.Cu") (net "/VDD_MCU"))
 (via (at 10.8 30.7) (size 0.6) (drill 0.3) (layers "F.Cu" "B.Cu") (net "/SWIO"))
 (segment (start 9.8 30.3) (end 10.4 30.3) (width 0.15) (layer "B.Cu") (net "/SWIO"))
 (segment (start 10.4 30.3) (end 10.8 30.7) (width 0.15) (layer "B.Cu") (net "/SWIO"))
 (via (at 10 31.9) (size 0.6) (drill 0.3) (layers "F.Cu" "B.Cu") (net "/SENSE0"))
 (segment (start 9.1 31) (end 9.1 31.1) (width 0.15) (layer "B.Cu") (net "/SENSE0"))
 (segment (start 9.1 31.1) (end 10 31.9) (width 0.15) (layer "B.Cu") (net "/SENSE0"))
 (via (at 7.8 31.9) (size 0.6) (drill 0.3) (layers "F.Cu" "B.Cu") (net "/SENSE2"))
 (segment (start 8.3 31.4) (end 7.8 31.9) (width 0.15) (layer "B.Cu") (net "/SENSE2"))
 (segment (start 8.3 31) (end 8.3 31.4) (width 0.15) (layer "B.Cu") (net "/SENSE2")))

